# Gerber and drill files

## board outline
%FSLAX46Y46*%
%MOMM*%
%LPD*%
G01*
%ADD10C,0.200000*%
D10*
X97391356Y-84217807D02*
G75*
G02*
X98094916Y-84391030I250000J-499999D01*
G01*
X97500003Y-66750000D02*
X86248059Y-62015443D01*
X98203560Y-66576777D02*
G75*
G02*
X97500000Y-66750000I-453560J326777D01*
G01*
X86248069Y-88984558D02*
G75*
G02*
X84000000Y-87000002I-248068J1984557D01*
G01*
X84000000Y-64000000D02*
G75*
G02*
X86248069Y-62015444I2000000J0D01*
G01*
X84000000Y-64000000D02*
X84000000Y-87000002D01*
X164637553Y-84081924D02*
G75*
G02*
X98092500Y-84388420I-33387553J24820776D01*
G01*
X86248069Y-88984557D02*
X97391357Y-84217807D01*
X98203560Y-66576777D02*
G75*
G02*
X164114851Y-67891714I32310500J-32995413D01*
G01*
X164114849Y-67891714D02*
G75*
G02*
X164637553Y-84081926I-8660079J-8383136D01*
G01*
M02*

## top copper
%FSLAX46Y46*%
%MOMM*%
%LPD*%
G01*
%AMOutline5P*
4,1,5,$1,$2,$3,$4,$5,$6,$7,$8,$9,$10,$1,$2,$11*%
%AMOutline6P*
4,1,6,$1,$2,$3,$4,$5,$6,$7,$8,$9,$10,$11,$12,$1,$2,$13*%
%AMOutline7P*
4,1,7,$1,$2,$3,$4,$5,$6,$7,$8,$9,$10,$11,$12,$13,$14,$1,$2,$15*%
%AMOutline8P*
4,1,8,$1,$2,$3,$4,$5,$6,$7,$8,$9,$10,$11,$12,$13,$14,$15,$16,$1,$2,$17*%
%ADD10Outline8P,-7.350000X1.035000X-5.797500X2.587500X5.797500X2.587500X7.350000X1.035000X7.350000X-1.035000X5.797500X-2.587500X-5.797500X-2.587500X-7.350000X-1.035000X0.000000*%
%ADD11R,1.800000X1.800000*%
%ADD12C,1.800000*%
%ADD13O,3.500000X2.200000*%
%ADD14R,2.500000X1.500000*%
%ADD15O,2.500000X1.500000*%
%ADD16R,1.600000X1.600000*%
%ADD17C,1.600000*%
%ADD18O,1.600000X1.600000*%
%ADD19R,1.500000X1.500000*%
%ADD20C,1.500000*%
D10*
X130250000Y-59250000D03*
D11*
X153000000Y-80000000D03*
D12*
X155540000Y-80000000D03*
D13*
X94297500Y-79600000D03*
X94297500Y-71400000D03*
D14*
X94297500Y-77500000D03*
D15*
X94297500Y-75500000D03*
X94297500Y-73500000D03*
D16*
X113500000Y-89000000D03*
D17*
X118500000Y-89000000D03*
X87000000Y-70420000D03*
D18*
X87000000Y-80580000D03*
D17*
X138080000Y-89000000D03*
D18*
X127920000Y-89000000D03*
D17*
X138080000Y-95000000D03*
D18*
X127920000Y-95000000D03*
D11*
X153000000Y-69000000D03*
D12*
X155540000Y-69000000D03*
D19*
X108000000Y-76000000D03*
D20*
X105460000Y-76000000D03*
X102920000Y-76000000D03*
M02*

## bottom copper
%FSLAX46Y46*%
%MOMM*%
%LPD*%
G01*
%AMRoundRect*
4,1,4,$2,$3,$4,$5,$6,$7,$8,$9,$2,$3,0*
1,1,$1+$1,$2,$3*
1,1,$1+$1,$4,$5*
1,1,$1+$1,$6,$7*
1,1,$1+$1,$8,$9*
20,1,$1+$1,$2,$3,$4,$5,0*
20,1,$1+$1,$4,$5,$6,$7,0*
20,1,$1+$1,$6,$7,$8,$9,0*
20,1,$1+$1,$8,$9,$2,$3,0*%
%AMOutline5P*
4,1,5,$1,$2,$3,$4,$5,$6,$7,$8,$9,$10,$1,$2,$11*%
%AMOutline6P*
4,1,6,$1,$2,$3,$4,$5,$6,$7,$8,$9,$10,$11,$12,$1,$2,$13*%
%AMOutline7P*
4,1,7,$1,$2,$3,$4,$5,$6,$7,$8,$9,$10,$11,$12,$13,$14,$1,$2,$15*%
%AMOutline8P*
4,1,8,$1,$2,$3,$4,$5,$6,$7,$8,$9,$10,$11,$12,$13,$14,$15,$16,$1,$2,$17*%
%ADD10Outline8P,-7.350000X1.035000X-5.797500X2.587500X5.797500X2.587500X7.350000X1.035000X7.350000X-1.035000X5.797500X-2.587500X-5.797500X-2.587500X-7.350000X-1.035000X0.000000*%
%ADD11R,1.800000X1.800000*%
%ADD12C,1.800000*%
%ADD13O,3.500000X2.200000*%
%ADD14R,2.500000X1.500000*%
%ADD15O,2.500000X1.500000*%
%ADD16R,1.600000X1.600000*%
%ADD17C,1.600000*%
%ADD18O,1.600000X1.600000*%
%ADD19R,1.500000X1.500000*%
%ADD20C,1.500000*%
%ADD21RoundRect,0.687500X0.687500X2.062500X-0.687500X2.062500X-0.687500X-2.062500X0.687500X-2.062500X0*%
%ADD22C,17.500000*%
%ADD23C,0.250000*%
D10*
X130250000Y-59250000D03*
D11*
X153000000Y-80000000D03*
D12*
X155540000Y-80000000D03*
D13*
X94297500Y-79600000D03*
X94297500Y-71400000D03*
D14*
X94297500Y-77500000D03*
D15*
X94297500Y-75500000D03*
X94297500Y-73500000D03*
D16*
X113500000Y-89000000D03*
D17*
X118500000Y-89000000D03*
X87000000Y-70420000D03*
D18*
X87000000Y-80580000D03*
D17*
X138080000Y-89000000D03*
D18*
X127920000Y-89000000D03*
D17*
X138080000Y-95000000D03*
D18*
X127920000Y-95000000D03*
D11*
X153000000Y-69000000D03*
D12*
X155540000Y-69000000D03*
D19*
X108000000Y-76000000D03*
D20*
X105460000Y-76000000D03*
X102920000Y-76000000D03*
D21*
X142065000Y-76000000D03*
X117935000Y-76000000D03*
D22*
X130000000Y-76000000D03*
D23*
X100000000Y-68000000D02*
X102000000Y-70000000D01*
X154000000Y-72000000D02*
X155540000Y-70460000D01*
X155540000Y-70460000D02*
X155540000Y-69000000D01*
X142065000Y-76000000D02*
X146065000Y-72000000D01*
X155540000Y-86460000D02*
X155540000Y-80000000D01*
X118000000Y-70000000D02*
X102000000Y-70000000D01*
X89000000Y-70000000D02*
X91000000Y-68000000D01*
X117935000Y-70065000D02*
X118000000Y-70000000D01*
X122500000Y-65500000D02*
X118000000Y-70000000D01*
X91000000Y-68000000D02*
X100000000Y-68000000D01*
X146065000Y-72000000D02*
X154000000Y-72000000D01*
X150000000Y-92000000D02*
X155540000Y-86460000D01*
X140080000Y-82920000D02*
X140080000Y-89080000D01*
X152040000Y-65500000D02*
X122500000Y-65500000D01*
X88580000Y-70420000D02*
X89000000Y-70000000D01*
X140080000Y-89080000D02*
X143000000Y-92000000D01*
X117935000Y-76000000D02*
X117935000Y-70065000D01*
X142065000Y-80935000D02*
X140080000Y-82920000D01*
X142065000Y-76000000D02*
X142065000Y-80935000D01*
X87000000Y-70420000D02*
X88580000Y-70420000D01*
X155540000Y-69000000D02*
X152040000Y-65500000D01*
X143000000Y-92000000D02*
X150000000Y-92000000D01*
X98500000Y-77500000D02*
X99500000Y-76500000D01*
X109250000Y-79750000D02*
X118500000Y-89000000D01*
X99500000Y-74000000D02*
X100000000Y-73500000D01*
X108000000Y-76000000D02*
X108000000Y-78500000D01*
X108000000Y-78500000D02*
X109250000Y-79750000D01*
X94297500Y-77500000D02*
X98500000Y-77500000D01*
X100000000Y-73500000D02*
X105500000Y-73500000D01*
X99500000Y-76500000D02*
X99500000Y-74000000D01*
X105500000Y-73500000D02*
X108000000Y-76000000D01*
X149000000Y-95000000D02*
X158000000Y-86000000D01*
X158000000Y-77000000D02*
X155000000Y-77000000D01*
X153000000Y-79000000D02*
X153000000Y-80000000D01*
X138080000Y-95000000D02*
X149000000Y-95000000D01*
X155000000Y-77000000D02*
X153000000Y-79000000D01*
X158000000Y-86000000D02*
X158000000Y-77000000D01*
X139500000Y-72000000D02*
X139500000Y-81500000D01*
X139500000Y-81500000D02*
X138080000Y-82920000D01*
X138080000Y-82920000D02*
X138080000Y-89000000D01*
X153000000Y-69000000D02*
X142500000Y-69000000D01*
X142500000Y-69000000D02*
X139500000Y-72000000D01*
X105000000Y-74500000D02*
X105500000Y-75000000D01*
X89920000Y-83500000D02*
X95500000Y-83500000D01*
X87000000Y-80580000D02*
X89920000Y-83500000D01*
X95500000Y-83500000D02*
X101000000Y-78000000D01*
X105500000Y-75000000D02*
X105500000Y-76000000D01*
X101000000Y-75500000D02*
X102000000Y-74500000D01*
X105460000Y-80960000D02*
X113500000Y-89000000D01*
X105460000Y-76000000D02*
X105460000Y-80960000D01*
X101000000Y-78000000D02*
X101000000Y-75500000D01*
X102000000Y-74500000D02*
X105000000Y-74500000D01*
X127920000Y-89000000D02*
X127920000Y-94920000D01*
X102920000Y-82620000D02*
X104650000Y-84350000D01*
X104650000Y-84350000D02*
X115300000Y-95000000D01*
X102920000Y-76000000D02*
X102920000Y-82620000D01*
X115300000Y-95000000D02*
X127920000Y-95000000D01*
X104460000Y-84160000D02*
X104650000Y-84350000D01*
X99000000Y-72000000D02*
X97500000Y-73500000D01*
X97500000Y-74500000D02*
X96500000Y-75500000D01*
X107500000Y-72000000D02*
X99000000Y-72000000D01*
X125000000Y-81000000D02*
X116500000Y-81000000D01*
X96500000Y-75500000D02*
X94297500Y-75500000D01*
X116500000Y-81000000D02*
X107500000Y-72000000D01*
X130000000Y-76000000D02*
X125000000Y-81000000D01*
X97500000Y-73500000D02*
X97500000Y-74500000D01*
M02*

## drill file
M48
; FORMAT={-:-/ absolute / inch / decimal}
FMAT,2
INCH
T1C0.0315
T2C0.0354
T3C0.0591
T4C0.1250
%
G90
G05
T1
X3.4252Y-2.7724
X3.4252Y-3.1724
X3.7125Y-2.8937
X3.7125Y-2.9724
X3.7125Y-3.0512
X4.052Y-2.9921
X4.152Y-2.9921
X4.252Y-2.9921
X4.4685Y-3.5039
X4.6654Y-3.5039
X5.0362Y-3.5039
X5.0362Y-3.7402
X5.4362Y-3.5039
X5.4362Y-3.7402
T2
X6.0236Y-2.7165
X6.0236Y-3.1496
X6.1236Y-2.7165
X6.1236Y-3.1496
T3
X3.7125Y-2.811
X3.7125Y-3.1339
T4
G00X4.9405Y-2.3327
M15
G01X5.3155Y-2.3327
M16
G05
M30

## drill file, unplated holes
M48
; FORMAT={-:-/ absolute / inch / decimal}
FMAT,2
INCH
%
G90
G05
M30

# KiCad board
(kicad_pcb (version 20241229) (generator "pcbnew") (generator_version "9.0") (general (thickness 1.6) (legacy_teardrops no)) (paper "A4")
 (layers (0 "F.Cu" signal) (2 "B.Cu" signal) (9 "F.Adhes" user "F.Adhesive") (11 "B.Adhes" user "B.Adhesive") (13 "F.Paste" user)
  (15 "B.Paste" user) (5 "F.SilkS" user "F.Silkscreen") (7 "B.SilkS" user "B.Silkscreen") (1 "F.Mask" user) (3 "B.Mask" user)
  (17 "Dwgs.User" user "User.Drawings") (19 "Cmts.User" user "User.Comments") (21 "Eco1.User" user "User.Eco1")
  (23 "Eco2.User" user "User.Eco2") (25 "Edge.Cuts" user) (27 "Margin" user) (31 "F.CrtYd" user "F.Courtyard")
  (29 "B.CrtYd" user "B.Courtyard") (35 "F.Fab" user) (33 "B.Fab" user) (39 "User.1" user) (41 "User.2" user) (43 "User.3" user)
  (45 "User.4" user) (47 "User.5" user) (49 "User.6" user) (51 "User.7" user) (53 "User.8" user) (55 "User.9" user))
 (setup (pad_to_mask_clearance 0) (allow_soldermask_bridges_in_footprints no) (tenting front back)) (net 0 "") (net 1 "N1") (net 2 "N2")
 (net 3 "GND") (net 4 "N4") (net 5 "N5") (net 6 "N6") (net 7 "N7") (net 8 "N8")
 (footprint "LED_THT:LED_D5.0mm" (layer "F.Cu") (at 153 80)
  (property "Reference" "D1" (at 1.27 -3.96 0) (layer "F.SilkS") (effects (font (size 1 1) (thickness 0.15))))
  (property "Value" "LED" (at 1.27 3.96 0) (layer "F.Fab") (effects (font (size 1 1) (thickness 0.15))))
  (pad "1" thru_hole rect (at 0 0) (size 1.8 1.8) (drill 0.9) (layers "*.Cu" "*.Mask") (remove_unused_layers no) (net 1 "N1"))
  (pad "2" thru_hole circle (at 2.54 0) (size 1.8 1.8) (drill 0.9) (layers "*.Cu" "*.Mask") (remove_unused_layers no) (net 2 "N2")))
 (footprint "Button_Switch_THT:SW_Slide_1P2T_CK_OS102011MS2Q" (layer "F.Cu") (at 94.2975 77.5 90)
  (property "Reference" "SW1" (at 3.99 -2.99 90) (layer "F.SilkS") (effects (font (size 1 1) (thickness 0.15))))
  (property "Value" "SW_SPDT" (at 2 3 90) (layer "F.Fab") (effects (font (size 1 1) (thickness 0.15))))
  (pad "" thru_hole oval (at -2.1 0 90) (size 2.2 3.5) (drill 1.5) (layers "*.Cu" "*.Mask") (remove_unused_layers no))
  (pad "" thru_hole oval (at 6.1 0 90) (size 2.2 3.5) (drill 1.5) (layers "*.Cu" "*.Mask") (remove_unused_layers no))
  (pad "1" thru_hole rect (at 0 0 90) (size 1.5 2.5) (drill 0.8) (layers "*.Cu" "*.Mask") (remove_unused_layers no) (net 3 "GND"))
  (pad "2" thru_hole oval (at 2 0 90) (size 1.5 2.5) (drill 0.8) (layers "*.Cu" "*.Mask") (remove_unused_layers no) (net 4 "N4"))
  (pad "3" thru_hole oval (at 4 0 90) (size 1.5 2.5) (drill 0.8) (layers "*.Cu" "*.Mask") (remove_unused_layers no) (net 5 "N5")))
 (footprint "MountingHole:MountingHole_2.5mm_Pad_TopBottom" (layer "F.Cu") (at 130.25 59.25)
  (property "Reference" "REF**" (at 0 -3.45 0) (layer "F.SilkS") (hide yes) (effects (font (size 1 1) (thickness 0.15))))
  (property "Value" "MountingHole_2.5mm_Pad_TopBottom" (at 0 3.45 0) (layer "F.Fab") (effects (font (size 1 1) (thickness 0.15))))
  (pad "1" thru_hole roundrect (at 0 0) (size 14.7 5.175) (drill oval 12.7 3.175) (layers "*.Cu" "*.Mask") (remove_unused_layers no)
   (roundrect_rratio 0) (chamfer_ratio 0.3) (chamfer top_left top_right bottom_left bottom_right) (zone_connect 2)))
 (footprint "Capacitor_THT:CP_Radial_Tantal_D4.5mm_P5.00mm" (layer "F.Cu") (at 113.5 89)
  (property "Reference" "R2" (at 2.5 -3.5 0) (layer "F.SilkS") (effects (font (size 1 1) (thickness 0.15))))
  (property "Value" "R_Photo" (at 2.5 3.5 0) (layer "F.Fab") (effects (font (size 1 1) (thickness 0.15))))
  (pad "1" thru_hole rect (at 0 0) (size 1.6 1.6) (drill 0.8) (layers "*.Cu" "*.Mask") (remove_unused_layers no) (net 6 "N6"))
  (pad "2" thru_hole circle (at 5 0) (size 1.6 1.6) (drill 0.8) (layers "*.Cu" "*.Mask") (remove_unused_layers no) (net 3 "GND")))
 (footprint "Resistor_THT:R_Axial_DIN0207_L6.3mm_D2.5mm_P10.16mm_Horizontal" (layer "F.Cu") (at 87 70.42 -90)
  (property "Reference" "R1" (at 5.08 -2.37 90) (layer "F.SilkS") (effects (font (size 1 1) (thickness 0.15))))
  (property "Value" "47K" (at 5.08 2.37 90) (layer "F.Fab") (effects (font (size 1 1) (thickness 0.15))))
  (pad "1" thru_hole circle (at 0 0 270) (size 1.6 1.6) (drill 0.8) (layers "*.Cu" "*.Mask") (remove_unused_layers no) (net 2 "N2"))
  (pad "2" thru_hole oval (at 10.16 0 270) (size 1.6 1.6) (drill 0.8) (layers "*.Cu" "*.Mask") (remove_unused_layers no) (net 6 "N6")))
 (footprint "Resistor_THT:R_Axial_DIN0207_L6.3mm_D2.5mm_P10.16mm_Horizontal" (layer "F.Cu") (at 138.08 89 180)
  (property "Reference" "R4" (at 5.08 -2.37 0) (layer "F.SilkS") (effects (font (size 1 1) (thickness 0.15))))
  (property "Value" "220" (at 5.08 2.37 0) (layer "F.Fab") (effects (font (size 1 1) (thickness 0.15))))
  (pad "1" thru_hole circle (at 0 0 180) (size 1.6 1.6) (drill 0.8) (layers "*.Cu" "*.Mask") (remove_unused_layers no) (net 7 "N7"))
  (pad "2" thru_hole oval (at 10.16 0 180) (size 1.6 1.6) (drill 0.8) (layers "*.Cu" "*.Mask") (remove_unused_layers no) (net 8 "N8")))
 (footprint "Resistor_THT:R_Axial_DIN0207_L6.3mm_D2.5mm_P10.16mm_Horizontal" (layer "F.Cu") (at 138.08 95 180)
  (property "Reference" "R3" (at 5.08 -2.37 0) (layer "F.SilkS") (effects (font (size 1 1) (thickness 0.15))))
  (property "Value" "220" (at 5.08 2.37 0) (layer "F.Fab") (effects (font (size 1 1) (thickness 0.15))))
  (pad "1" thru_hole circle (at 0 0 180) (size 1.6 1.6) (drill 0.8) (layers "*.Cu" "*.Mask") (remove_unused_layers no) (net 1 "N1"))
  (pad "2" thru_hole oval (at 10.16 0 180) (size 1.6 1.6) (drill 0.8) (layers "*.Cu" "*.Mask") (remove_unused_layers no) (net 8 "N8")))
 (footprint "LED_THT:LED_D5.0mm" (layer "F.Cu") (at 153 69)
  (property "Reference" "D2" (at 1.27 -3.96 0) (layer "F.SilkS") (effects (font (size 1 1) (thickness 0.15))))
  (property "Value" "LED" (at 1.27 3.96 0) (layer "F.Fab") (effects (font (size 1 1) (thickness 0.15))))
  (pad "1" thru_hole rect (at 0 0) (size 1.8 1.8) (drill 0.9) (layers "*.Cu" "*.Mask") (remove_unused_layers no) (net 7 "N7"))
  (pad "2" thru_hole circle (at 2.54 0) (size 1.8 1.8) (drill 0.9) (layers "*.Cu" "*.Mask") (remove_unused_layers no) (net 2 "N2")))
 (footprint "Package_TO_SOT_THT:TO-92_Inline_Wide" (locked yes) (layer "F.Cu") (at 108 76 180)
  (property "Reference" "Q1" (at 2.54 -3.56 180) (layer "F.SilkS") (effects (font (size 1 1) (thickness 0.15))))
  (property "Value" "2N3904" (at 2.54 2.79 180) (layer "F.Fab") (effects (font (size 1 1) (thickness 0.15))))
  (pad "1" thru_hole rect (at 0 0 180) (size 1.5 1.5) (drill 0.8) (layers "*.Cu" "*.Mask") (remove_unused_layers no) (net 3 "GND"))
  (pad "2" thru_hole circle (at 2.54 0 180) (size 1.5 1.5) (drill 0.8) (layers "*.Cu" "*.Mask") (remove_unused_layers no) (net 6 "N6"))
  (pad "3" thru_hole circle (at 5.08 0 180) (size 1.5 1.5) (drill 0.8) (layers "*.Cu" "*.Mask") (remove_unused_layers no) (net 8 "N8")))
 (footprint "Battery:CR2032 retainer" (layer "B.Cu") (at 130 76 180)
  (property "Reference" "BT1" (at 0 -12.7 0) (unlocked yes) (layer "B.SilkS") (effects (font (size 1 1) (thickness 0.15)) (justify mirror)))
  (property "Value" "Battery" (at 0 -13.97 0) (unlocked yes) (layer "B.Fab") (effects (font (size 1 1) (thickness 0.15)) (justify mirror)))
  (pad "1" smd roundrect (at -12.065 0 180) (size 2.75 5.5) (layers "B.Cu" "B.Mask" "B.Paste") (roundrect_rratio 0.25) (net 2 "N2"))
  (pad "1" smd roundrect (at 12.065 0 180) (size 2.75 5.5) (layers "B.Cu" "B.Mask" "B.Paste") (roundrect_rratio 0.25) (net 2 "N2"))
  (pad "2" smd circle (at 0 0 180) (size 17.5 17.5) (layers "B.Cu" "B.Mask" "B.Paste") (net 4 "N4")))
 (gr_arc (start 97.391356 84.217807) (mid 97.775 84.175) (end 98.094916 84.39103) (stroke (width 0.2) (type default)) (layer "Edge.Cuts"))
 (gr_line (start 97.500003 66.75) (end 86.248059 62.015443) (stroke (width 0.2) (type solid)) (layer "Edge.Cuts"))
 (gr_line (start 84 64) (end 84 87.000002) (stroke (width 0.2) (type solid)) (layer "Edge.Cuts"))
 (gr_arc (start 164.637553 84.081924) (mid 131.441614 100.863587) (end 98.092499 84.38842) (stroke (width 0.2) (type solid))
  (layer "Edge.Cuts"))
 (gr_line (start 86.248069 88.984557) (end 97.391357 84.217807) (stroke (width 0.2) (type solid)) (layer "Edge.Cuts"))
 (gr_arc (start 98.20356 66.576777) (mid 97.883644 66.792807) (end 97.5 66.75) (stroke (width 0.2) (type default)) (layer "Edge.Cuts"))
 (gr_arc (start 84 64) (mid 84.676395 62.500644) (end 86.248069 62.015444) (stroke (width 0.2) (type default)) (layer "Edge.Cuts"))
 (gr_arc (start 86.248069 88.984558) (mid 84.676395 88.499358) (end 84 87.000002) (stroke (width 0.2) (type default)) (layer "Edge.Cuts"))
 (gr_arc (start 98.20356 66.576777) (mid 131.435188 53.400584) (end 164.114851 67.891714) (stroke (width 0.2) (type solid))
  (layer "Edge.Cuts"))
 (gr_arc (start 164.114849 67.891714) (mid 167.501457 75.885921) (end 164.637553 84.081926) (stroke (width 0.2) (type solid))
  (layer "Edge.Cuts"))
 (segment (start 100 68) (end 102 70) (width 0.25) (layer "B.Cu") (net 2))
 (segment (start 154 72) (end 155.54 70.46) (width 0.25) (layer "B.Cu") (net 2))
 (segment (start 155.54 70.46) (end 155.54 69) (width 0.25) (layer "B.Cu") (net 2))
 (segment (start 142.065 76) (end 146.065 72) (width 0.25) (layer "B.Cu") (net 2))
 (segment (start 155.54 86.46) (end 155.54 80) (width 0.25) (layer "B.Cu") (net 2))
 (segment (start 118 70) (end 102 70) (width 0.25) (layer "B.Cu") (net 2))
 (segment (start 89 70) (end 91 68) (width 0.25) (layer "B.Cu") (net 2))
 (segment (start 117.935 70.065) (end 118 70) (width 0.25) (layer "B.Cu") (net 2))
 (segment (start 122.5 65.5) (end 118 70) (width 0.25) (layer "B.Cu") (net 2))
 (segment (start 91 68) (end 100 68) (width 0.25) (layer "B.Cu") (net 2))
 (segment (start 146.065 72) (end 154 72) (width 0.25) (layer "B.Cu") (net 2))
 (segment (start 150 92) (end 155.54 86.46) (width 0.25) (layer "B.Cu") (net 2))
 (segment (start 140.08 82.92) (end 140.08 89.08) (width 0.25) (layer "B.Cu") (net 2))
 (segment (start 152.04 65.5) (end 122.5 65.5) (width 0.25) (layer "B.Cu") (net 2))
 (segment (start 88.58 70.42) (end 89 70) (width 0.25) (layer "B.Cu") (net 2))
 (segment (start 140.08 89.08) (end 143 92) (width 0.25) (layer "B.Cu") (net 2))
 (segment (start 117.935 76) (end 117.935 70.065) (width 0.25) (layer "B.Cu") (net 2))
 (segment (start 142.065 80.935) (end 140.08 82.92) (width 0.25) (layer "B.Cu") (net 2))
 (segment (start 142.065 76) (end 142.065 80.935) (width 0.25) (layer "B.Cu") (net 2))
 (segment (start 87 70.42) (end 88.58 70.42) (width 0.25) (layer "B.Cu") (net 2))
 (segment (start 155.54 69) (end 152.04 65.5) (width 0.25) (layer "B.Cu") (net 2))
 (segment (start 143 92) (end 150 92) (width 0.25) (layer "B.Cu") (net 2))
 (segment (start 98.5 77.5) (end 99.5 76.5) (width 0.25) (layer "B.Cu") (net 3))
 (segment (start 109.25 79.75) (end 118.5 89) (width 0.25) (layer "B.Cu") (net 3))
 (segment (start 99.5 74) (end 100 73.5) (width 0.25) (layer "B.Cu") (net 3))
 (segment (start 108 76) (end 108 78.5) (width 0.25) (layer "B.Cu") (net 3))
 (segment (start 108 78.5) (end 109.25 79.75) (width 0.25) (layer "B.Cu") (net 3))
 (segment (start 94.2975 77.5) (end 98.5 77.5) (width 0.25) (layer "B.Cu") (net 3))
 (segment (start 100 73.5) (end 105.5 73.5) (width 0.25) (layer "B.Cu") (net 3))
 (segment (start 99.5 76.5) (end 99.5 74) (width 0.25) (layer "B.Cu") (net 3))
 (segment (start 105.5 73.5) (end 108 76) (width 0.25) (layer "B.Cu") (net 3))
 (segment (start 149 95) (end 158 86) (width 0.25) (layer "B.Cu") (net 1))
 (segment (start 158 77) (end 155 77) (width 0.25) (layer "B.Cu") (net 1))
 (segment (start 153 79) (end 153 80) (width 0.25) (layer "B.Cu") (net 1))
 (segment (start 138.08 95) (end 149 95) (width 0.25) (layer "B.Cu") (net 1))
 (segment (start 155 77) (end 153 79) (width 0.25) (layer "B.Cu") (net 1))
 (segment (start 158 86) (end 158 77) (width 0.25) (layer "B.Cu") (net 1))
 (segment (start 139.5 72) (end 139.5 81.5) (width 0.25) (layer "B.Cu") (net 7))
 (segment (start 139.5 81.5) (end 138.08 82.92) (width 0.25) (layer "B.Cu") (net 7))
 (segment (start 138.08 82.92) (end 138.08 89) (width 0.25) (layer "B.Cu") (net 7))
 (segment (start 153 69) (end 142.5 69) (width 0.25) (layer "B.Cu") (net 7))
 (segment (start 142.5 69) (end 139.5 72) (width 0.25) (layer "B.Cu") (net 7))
 (segment (start 105 74.5) (end 105.5 75) (width 0.25) (layer "B.Cu") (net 6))
 (segment (start 89.92 83.5) (end 95.5 83.5) (width 0.25) (layer "B.Cu") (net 6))
 (segment (start 87 80.58) (end 89.92 83.5) (width 0.25) (layer "B.Cu") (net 6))
 (segment (start 95.5 83.5) (end 101 78) (width 0.25) (layer "B.Cu") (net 6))
 (segment (start 105.5 75) (end 105.5 76) (width 0.25) (layer "B.Cu") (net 6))
 (segment (start 101 75.5) (end 102 74.5) (width 0.25) (layer "B.Cu") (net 6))
 (segment (start 105.46 80.96) (end 113.5 89) (width 0.25) (layer "B.Cu") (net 6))
 (segment (start 105.46 76) (end 105.46 80.96) (width 0.25) (layer "B.Cu") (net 6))
 (segment (start 101 78) (end 101 75.5) (width 0.25) (layer "B.Cu") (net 6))
 (segment (start 102 74.5) (end 105 74.5) (width 0.25) (layer "B.Cu") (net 6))
 (segment (start 127.92 89) (end 127.92 94.92) (width 0.25) (layer "B.Cu") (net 8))
 (segment (start 102.92 82.62) (end 104.65 84.35) (width 0.25) (layer "B.Cu") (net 8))
 (segment (start 104.65 84.35) (end 115.3 95) (width 0.25) (layer "B.Cu") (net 8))
 (segment (start 102.92 76) (end 102.92 82.62) (width 0.25) (layer "B.Cu") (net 8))
 (segment (start 115.3 95) (end 127.92 95) (width 0.25) (layer "B.Cu") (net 8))
 (segment (start 104.46 84.16) (end 104.65 84.35) (width 0.25) (layer "B.Cu") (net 8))
 (segment (start 99 72) (end 97.5 73.5) (width 0.25) (layer "B.Cu") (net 4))
 (segment (start 97.5 74.5) (end 96.5 75.5) (width 0.25) (layer "B.Cu") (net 4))
 (segment (start 107.5 72) (end 99 72) (width 0.25) (layer "B.Cu") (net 4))
 (segment (start 125 81) (end 116.5 81) (width 0.25) (layer "B.Cu") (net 4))
 (segment (start 96.5 75.5) (end 94.2975 75.5) (width 0.25) (layer "B.Cu") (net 4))
 (segment (start 116.5 81) (end 107.5 72) (width 0.25) (layer "B.Cu") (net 4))
 (segment (start 130 76) (end 125 81) (width 0.25) (layer "B.Cu") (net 4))
 (segment (start 97.5 73.5) (end 97.5 74.5) (width 0.25) (layer "B.Cu") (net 4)))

